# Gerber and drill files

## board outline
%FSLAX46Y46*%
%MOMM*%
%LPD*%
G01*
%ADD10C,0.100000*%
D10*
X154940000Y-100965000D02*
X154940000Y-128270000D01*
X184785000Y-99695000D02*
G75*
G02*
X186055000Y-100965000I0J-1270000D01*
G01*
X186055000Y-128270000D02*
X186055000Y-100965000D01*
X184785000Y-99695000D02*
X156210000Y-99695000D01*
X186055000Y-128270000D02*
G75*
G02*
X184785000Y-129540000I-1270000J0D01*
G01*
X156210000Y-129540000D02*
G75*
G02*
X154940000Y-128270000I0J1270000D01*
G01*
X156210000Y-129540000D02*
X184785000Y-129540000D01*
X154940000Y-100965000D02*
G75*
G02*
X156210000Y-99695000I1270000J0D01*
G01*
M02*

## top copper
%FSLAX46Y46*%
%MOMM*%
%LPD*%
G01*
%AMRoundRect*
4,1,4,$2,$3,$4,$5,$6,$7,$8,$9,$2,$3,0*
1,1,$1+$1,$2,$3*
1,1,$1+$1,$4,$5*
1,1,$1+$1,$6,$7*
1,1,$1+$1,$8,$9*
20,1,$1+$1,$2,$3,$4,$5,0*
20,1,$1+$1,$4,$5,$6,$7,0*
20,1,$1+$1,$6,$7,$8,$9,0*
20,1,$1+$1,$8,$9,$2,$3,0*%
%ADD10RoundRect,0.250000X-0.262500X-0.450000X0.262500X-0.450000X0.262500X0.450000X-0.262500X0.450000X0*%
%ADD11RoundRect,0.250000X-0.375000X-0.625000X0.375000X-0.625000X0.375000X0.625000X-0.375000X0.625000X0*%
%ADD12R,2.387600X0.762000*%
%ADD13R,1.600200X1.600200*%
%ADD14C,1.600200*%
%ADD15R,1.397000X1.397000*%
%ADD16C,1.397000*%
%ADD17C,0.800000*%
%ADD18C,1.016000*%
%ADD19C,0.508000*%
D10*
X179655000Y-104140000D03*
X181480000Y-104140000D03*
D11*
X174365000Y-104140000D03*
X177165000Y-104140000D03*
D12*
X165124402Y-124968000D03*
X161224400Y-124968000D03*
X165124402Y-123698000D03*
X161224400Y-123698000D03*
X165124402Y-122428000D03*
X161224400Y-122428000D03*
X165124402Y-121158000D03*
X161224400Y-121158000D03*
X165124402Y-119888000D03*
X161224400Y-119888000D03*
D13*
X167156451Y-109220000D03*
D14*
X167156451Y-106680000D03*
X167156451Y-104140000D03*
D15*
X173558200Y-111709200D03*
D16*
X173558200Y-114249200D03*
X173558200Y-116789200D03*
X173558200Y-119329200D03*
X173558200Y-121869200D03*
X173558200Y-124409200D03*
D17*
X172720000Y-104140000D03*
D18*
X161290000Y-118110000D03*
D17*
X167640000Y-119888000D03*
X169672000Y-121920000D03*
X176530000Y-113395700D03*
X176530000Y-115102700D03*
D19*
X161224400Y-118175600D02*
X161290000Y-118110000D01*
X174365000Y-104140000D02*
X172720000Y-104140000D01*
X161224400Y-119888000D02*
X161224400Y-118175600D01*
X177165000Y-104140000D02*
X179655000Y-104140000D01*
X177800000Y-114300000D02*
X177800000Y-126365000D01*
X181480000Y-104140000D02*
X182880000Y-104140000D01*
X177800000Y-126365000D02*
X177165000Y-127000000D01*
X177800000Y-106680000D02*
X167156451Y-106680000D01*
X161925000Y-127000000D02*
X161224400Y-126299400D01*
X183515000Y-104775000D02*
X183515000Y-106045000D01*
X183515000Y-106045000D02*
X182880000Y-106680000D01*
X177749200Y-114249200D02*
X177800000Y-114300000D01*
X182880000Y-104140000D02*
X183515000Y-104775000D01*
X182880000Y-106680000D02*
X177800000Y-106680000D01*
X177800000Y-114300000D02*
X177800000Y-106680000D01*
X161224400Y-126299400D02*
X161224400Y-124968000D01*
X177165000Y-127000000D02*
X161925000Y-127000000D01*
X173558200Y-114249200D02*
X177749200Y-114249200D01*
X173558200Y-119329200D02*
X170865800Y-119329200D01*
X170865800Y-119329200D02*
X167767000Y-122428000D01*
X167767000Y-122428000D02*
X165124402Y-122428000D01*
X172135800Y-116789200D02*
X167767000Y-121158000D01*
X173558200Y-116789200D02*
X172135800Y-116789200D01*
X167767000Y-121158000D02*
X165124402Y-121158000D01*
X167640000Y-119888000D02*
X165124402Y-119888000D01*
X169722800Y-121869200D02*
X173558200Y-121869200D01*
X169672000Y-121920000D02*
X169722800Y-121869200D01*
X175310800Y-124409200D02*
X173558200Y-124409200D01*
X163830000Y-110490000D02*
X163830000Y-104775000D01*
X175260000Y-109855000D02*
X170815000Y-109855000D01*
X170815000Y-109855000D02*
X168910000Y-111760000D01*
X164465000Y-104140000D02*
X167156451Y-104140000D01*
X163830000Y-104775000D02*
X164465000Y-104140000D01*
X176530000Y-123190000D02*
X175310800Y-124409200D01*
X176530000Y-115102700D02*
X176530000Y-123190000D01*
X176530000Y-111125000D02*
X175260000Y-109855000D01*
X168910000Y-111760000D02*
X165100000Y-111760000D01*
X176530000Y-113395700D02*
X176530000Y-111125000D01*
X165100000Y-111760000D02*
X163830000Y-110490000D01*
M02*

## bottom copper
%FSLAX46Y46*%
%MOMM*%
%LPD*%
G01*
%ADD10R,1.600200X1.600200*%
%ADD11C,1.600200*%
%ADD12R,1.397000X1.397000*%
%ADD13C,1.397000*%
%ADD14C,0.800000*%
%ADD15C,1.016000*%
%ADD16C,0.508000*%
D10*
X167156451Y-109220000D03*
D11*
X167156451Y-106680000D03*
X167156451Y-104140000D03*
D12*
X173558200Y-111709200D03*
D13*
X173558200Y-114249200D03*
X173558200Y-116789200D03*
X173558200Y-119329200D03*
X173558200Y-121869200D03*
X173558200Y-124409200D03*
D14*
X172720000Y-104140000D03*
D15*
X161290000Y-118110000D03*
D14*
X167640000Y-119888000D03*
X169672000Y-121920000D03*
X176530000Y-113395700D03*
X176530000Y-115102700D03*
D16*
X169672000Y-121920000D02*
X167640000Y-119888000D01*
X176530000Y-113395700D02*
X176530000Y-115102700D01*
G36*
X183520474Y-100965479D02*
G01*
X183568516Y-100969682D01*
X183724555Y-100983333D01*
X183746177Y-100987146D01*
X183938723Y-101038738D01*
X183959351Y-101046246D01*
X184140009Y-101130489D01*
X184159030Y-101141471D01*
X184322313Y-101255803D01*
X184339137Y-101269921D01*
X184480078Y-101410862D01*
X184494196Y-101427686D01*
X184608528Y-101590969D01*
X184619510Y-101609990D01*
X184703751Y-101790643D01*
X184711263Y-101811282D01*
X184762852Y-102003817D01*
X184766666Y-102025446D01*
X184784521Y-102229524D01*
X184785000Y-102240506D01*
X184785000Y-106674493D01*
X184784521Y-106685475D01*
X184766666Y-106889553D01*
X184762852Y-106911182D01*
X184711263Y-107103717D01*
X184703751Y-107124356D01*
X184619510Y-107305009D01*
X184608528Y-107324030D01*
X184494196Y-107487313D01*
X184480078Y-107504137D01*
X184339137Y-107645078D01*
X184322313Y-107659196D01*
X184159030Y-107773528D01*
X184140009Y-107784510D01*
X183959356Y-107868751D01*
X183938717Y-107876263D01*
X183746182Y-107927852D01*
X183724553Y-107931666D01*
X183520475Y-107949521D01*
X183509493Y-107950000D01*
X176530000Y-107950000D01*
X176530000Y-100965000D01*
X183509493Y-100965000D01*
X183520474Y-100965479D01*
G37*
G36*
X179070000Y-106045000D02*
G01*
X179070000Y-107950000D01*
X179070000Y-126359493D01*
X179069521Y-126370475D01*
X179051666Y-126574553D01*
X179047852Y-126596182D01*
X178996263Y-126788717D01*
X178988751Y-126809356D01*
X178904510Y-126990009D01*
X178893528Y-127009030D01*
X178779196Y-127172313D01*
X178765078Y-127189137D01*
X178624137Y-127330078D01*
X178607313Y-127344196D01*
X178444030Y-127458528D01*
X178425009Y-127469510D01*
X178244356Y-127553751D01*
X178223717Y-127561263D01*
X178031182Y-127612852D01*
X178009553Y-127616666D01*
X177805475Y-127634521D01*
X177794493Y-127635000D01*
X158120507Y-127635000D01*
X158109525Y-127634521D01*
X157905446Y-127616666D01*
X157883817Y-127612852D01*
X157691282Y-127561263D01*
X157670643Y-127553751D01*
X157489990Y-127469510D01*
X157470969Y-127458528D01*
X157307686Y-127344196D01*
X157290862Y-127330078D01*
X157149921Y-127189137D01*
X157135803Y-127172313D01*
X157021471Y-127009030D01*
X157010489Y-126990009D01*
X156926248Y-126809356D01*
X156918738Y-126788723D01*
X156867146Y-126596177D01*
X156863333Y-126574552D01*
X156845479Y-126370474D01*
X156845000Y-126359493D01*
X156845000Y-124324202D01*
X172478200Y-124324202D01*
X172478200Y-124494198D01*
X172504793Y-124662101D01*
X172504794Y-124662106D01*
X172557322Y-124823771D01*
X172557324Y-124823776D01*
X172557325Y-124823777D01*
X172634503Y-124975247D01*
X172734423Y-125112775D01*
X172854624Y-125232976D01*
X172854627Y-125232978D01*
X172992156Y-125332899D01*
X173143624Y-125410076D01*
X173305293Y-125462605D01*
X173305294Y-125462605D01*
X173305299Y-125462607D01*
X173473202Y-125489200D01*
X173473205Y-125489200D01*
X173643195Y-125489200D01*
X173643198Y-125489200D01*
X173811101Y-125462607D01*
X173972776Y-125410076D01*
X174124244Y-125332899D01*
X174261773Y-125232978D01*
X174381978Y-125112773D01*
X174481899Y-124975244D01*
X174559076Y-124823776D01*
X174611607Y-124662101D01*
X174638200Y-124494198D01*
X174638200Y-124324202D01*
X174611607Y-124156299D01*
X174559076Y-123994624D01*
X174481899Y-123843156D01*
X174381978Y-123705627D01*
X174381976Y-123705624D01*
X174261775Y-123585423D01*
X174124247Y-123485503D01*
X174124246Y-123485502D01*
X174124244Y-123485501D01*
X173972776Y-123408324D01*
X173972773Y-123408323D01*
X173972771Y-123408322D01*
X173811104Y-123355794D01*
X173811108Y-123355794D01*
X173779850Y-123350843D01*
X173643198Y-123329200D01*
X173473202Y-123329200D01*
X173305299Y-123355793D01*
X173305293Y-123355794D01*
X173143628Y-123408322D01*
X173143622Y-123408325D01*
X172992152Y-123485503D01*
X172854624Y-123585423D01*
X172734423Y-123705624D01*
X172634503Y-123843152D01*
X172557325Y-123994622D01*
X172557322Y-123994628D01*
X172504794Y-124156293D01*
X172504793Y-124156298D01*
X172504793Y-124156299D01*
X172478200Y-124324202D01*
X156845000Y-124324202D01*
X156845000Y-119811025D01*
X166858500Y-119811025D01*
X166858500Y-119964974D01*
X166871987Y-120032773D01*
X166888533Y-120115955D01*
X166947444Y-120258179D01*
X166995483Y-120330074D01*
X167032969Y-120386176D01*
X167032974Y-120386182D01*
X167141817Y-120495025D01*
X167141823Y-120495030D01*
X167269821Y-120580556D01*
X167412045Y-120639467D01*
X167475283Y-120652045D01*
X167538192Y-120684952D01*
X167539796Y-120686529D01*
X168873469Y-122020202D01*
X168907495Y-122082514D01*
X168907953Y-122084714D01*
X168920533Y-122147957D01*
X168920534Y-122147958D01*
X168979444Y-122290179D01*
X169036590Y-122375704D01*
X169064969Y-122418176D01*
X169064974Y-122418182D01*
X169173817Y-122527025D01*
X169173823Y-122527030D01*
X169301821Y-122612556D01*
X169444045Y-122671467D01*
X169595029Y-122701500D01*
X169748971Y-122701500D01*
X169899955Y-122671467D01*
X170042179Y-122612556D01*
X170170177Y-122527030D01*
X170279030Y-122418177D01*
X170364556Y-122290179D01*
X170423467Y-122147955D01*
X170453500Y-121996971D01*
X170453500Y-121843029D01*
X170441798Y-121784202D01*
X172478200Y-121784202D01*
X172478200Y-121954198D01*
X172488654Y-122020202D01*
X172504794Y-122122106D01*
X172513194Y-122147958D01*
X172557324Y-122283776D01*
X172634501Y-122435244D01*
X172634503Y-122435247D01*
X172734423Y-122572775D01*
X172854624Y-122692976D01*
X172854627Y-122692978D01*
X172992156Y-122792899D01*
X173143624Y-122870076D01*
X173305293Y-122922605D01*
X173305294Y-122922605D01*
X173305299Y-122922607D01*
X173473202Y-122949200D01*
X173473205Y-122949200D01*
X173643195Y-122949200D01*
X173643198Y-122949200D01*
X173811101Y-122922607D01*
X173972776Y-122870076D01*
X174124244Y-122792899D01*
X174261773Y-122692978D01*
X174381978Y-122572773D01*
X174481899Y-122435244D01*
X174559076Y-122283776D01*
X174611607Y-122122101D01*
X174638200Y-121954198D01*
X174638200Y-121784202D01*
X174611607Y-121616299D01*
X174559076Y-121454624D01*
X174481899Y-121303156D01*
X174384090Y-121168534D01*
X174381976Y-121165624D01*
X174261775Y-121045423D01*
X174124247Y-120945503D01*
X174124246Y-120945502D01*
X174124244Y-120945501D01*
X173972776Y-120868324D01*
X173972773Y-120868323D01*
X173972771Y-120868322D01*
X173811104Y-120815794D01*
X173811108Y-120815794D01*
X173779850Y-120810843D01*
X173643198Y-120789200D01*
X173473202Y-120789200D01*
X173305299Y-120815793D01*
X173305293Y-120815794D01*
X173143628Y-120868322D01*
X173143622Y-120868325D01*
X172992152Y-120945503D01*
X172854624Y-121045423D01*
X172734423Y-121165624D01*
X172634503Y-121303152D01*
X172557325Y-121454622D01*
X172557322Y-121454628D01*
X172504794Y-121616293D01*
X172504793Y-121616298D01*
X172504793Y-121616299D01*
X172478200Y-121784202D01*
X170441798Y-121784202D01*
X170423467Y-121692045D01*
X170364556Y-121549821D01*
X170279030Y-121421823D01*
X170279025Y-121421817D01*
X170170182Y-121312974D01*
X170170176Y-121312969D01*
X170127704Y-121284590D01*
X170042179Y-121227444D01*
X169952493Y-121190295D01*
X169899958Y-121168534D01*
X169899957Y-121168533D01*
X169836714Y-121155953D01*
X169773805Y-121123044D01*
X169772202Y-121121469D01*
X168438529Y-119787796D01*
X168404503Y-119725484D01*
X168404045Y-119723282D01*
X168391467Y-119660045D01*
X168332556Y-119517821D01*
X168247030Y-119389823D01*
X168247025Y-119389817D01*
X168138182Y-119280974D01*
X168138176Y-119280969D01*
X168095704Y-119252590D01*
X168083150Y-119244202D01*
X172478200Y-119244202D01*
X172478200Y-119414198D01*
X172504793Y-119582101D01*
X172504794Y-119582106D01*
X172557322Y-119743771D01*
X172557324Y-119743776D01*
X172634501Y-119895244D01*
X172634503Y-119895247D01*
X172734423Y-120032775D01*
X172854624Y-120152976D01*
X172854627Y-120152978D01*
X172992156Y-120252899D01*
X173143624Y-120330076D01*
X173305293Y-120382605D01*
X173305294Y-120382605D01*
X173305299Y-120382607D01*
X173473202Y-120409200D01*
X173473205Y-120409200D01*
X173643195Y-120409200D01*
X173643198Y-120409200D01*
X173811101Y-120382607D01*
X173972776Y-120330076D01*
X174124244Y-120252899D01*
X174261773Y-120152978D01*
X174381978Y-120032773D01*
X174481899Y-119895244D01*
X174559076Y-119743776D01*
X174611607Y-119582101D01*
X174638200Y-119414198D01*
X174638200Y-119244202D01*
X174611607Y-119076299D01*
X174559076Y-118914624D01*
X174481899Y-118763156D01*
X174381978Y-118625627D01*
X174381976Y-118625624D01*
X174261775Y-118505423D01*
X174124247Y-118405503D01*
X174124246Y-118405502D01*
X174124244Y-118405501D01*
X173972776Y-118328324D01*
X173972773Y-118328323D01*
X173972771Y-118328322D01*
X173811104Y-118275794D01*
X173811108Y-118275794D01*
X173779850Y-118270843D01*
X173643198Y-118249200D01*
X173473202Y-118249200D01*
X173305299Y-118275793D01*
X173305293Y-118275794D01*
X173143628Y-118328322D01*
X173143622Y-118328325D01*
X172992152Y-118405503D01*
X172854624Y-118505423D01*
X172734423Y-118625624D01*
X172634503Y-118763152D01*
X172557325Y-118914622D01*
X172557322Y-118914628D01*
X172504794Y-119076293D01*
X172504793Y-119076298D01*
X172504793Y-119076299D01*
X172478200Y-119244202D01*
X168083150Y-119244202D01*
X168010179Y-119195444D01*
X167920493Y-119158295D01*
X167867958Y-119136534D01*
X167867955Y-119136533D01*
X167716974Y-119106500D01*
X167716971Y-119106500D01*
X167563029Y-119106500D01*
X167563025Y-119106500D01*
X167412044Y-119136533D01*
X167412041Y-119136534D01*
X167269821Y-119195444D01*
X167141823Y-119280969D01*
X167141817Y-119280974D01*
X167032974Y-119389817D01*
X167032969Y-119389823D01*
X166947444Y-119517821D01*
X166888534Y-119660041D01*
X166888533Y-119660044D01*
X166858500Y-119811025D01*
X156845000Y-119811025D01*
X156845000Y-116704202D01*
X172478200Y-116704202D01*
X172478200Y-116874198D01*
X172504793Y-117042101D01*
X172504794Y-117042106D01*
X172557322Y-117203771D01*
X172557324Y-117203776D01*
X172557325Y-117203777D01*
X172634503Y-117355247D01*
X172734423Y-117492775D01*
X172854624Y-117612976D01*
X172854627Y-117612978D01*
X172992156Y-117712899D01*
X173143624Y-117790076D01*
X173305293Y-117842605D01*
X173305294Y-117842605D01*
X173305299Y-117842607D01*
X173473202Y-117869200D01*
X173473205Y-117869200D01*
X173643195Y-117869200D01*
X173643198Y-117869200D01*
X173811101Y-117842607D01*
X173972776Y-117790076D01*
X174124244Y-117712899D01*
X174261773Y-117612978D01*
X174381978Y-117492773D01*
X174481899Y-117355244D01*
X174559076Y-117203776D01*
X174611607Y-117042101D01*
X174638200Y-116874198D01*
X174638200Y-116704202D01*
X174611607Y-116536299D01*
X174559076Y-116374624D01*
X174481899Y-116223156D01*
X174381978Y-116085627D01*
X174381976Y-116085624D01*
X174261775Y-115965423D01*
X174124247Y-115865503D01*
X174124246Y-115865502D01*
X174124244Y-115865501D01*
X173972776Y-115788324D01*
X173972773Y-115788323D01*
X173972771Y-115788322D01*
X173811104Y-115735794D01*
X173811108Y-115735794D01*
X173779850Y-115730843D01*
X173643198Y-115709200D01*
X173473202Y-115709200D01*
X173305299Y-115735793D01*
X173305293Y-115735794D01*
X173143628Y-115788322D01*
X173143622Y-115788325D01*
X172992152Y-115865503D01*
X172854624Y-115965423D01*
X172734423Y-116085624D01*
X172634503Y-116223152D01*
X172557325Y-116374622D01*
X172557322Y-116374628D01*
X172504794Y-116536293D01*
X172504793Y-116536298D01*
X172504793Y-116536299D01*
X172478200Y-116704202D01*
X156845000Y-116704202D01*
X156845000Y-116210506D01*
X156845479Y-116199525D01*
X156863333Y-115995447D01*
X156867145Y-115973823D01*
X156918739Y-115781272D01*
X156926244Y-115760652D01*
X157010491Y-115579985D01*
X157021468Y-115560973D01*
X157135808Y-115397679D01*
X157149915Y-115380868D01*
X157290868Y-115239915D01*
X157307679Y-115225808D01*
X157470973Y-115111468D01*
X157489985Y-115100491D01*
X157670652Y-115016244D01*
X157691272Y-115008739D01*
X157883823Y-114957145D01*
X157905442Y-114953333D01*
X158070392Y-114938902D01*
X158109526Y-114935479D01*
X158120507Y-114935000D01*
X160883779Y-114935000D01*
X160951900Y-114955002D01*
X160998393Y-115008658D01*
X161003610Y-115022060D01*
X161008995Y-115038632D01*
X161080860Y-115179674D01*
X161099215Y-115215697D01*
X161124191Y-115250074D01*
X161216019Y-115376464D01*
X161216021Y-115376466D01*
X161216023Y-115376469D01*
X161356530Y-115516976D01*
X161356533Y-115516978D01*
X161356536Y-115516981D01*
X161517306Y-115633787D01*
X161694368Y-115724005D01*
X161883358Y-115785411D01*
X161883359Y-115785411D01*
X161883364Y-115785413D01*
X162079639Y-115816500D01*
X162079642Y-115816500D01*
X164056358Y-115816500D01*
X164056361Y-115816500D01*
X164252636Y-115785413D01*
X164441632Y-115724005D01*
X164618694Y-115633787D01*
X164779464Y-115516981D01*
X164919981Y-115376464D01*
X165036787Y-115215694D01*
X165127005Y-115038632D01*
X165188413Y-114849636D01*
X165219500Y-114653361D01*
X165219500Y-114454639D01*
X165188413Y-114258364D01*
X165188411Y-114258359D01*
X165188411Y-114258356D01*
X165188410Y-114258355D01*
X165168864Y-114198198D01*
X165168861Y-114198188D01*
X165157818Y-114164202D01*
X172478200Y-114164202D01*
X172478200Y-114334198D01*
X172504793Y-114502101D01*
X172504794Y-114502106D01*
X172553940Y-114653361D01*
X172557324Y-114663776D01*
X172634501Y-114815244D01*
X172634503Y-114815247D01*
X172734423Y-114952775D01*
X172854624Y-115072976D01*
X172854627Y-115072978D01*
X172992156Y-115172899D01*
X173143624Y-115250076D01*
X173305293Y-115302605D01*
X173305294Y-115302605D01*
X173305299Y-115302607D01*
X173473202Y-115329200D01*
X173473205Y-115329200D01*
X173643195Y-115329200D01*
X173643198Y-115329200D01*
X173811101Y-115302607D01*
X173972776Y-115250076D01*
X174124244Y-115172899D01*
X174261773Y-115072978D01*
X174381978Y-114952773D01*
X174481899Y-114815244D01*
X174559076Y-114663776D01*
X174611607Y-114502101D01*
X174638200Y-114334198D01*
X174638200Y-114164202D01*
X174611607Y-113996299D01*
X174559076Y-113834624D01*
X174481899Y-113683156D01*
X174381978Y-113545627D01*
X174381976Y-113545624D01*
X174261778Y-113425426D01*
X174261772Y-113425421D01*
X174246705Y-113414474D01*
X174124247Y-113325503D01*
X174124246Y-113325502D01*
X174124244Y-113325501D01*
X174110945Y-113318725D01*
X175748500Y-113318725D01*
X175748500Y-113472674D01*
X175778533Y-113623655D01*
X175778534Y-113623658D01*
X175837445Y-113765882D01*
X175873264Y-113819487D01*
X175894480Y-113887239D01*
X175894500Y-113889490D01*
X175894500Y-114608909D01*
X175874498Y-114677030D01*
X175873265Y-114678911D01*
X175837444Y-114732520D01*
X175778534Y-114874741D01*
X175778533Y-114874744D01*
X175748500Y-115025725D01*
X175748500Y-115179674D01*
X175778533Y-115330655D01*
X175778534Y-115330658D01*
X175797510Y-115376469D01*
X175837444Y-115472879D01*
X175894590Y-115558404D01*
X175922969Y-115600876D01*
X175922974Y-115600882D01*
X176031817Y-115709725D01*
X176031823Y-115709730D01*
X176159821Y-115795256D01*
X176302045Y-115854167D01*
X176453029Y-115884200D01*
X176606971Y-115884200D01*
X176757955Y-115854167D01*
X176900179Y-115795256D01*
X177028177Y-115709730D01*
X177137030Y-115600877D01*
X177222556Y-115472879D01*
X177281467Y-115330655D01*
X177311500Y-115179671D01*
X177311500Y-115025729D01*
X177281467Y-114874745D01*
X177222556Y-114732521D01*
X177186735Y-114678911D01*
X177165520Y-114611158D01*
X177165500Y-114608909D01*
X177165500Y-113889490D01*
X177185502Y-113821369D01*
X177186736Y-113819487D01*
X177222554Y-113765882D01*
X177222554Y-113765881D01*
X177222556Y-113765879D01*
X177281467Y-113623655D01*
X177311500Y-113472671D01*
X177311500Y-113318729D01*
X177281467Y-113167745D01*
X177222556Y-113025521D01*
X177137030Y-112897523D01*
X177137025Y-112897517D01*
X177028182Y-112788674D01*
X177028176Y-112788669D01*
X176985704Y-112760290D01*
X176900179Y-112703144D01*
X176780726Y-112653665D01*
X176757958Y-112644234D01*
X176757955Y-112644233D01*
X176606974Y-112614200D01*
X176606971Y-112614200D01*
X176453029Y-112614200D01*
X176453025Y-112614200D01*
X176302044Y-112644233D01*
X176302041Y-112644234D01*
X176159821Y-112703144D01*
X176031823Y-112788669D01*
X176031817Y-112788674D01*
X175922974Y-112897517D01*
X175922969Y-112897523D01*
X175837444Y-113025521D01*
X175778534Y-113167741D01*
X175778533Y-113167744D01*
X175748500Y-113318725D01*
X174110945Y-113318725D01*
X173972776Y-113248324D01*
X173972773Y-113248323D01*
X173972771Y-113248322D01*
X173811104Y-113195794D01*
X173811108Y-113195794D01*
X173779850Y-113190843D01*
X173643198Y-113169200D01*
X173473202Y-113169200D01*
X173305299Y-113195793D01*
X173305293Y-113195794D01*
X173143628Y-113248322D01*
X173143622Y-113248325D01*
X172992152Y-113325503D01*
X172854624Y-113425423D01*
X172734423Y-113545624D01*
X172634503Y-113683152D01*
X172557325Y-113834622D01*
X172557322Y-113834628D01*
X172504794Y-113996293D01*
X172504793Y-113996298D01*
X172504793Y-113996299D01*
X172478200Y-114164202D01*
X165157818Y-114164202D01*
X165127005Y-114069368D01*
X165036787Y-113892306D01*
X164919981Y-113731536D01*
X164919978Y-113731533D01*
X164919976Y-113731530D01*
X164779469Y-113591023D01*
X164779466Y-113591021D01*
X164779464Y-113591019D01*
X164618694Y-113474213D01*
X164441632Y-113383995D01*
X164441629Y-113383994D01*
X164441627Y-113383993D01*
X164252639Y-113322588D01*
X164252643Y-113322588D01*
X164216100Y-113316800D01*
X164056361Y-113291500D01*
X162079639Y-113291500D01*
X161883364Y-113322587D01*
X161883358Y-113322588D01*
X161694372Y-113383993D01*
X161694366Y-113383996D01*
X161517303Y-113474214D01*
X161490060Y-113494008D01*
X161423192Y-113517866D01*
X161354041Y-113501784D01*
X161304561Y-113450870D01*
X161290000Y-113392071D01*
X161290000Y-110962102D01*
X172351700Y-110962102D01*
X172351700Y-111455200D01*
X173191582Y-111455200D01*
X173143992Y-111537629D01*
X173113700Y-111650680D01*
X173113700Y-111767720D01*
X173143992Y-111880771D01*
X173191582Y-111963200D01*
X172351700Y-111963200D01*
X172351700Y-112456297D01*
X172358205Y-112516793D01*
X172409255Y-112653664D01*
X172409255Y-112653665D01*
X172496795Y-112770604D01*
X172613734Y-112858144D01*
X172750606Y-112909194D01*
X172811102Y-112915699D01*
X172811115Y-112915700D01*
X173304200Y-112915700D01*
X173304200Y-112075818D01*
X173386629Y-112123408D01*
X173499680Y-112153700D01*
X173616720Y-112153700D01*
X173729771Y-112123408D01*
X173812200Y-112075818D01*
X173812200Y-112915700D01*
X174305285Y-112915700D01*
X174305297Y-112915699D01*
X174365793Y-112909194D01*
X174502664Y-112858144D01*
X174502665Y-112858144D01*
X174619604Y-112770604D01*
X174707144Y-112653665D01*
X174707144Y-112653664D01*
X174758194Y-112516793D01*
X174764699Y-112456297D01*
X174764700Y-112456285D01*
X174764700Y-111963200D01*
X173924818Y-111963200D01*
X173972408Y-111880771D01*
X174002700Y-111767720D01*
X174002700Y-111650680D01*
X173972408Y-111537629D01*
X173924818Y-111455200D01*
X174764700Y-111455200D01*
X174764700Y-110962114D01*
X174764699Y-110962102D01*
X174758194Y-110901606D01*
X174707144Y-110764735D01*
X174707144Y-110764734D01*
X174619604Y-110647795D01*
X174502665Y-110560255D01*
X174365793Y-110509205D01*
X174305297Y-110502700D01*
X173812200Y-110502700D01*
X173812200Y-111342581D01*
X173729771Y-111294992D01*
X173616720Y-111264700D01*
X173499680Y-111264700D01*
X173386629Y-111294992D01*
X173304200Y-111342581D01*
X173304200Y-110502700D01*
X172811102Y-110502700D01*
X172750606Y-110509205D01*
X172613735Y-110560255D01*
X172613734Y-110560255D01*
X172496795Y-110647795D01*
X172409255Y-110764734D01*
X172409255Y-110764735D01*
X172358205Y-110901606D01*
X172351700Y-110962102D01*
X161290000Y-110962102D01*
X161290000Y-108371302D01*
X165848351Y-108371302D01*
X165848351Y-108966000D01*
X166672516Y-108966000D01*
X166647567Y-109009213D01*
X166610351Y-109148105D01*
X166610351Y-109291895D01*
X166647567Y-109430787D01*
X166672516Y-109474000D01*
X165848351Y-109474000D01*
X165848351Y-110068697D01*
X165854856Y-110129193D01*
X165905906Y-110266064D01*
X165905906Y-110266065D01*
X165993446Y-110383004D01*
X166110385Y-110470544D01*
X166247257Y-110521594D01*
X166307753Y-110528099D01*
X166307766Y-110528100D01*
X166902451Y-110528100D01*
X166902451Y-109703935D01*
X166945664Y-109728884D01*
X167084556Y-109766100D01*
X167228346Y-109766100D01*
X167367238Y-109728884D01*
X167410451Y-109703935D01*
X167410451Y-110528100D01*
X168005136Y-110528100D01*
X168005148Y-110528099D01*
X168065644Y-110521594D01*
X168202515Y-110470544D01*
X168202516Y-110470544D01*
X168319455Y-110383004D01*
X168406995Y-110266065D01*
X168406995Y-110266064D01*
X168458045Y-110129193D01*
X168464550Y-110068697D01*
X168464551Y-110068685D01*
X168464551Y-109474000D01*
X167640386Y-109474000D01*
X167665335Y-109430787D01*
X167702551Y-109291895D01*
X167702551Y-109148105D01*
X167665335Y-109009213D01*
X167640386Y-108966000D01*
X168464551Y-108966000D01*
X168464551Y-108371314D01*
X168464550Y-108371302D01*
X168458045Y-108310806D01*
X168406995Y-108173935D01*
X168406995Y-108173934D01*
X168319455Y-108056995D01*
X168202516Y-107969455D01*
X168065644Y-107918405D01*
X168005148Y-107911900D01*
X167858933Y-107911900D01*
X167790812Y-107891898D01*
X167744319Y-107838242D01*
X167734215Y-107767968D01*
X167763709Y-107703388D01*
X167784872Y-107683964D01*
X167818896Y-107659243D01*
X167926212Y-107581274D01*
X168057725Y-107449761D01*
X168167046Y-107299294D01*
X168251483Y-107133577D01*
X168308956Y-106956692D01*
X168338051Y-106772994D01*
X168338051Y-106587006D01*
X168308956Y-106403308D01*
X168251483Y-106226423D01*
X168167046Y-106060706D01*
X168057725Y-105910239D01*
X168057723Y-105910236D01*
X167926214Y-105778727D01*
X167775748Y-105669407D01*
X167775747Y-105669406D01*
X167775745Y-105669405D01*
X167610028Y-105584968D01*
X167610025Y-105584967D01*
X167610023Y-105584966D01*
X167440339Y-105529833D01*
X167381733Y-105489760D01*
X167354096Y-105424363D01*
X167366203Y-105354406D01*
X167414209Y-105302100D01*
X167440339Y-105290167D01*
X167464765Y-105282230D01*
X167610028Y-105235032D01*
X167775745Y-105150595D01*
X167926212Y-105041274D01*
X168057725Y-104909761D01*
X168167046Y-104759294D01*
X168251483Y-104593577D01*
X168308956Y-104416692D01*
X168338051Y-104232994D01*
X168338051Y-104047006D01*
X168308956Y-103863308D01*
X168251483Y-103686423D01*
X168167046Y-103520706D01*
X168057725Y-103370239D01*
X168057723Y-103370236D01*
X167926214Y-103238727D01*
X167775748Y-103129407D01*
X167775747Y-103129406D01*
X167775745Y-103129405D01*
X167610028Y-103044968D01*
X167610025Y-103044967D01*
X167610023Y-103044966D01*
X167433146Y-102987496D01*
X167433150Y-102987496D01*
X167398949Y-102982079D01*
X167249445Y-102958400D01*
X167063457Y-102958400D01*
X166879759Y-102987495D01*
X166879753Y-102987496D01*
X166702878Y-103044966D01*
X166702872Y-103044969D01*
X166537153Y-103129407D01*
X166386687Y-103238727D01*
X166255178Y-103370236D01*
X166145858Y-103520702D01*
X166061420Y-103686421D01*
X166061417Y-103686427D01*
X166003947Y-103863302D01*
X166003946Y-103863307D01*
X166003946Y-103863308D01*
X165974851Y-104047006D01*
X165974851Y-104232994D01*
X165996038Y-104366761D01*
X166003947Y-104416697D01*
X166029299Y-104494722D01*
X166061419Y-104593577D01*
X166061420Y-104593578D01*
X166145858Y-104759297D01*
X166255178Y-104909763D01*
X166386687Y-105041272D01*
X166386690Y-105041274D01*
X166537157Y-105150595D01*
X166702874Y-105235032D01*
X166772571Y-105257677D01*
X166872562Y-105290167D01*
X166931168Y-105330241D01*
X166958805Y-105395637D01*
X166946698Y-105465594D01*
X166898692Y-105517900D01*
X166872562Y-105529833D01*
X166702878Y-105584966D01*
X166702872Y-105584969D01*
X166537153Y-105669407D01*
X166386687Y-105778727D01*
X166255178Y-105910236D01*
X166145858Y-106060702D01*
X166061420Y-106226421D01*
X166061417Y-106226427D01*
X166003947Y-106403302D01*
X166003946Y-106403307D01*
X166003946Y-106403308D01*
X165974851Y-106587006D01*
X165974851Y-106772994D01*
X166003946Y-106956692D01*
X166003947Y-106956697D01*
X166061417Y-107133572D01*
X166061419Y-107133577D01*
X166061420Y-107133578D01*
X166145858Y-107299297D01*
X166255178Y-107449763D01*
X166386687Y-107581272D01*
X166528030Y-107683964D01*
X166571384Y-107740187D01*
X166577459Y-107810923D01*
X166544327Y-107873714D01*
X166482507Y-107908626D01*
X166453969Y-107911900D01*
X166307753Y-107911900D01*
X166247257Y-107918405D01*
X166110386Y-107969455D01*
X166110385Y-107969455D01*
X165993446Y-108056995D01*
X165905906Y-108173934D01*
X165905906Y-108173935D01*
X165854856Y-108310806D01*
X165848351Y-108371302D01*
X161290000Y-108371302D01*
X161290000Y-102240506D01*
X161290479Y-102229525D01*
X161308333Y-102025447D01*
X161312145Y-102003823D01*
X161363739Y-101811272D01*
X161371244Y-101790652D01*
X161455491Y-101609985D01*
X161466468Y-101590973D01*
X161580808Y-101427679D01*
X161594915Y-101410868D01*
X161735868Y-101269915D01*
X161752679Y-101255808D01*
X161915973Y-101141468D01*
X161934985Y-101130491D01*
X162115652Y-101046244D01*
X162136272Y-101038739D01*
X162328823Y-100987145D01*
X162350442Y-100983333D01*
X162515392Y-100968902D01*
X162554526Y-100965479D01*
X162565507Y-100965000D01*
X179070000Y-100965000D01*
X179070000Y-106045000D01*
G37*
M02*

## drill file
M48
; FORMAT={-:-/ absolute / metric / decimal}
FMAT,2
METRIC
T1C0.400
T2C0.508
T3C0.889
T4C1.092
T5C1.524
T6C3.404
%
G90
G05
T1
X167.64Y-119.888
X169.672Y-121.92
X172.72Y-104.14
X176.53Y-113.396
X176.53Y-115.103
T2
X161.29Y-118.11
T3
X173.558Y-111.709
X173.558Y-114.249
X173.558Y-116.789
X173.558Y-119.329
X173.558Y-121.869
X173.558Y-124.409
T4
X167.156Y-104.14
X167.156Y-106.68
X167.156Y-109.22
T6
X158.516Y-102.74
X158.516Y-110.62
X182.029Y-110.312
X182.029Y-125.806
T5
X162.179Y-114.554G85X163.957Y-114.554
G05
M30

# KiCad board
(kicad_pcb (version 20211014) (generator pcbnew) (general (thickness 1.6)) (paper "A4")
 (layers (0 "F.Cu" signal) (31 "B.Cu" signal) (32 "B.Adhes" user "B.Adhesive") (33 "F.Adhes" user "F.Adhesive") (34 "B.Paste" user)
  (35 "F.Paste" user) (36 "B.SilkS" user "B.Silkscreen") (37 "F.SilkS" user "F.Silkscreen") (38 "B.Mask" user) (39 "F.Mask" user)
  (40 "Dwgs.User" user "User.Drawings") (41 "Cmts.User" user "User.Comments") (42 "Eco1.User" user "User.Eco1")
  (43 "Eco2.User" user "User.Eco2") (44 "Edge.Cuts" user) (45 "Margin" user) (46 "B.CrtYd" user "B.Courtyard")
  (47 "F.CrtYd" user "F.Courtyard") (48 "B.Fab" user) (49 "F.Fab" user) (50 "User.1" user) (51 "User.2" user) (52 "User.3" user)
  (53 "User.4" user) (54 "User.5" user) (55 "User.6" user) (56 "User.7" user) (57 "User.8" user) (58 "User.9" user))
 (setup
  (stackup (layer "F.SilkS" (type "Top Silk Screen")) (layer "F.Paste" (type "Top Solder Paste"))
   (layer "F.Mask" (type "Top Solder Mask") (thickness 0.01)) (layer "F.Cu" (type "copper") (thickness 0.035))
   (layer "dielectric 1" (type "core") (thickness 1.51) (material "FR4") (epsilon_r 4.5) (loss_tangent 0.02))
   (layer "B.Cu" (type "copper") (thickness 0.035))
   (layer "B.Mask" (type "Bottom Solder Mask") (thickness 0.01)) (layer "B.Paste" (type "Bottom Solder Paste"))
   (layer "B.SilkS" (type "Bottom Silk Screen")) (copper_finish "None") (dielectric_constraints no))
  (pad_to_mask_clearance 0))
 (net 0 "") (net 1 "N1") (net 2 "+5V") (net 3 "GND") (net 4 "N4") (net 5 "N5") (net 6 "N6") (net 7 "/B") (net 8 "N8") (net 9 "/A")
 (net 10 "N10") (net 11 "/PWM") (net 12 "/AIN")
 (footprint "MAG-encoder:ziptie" (layer "F.Cu") (at 163.068 114.554)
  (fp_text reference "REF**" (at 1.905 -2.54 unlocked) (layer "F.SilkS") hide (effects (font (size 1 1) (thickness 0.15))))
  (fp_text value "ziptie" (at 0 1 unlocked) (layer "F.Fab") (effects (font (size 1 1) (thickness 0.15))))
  (pad "" np_thru_hole oval (at 0 0) (size 3.302 1.524) (drill oval 3.302 1.524) (layers F&B.Cu *.Mask)))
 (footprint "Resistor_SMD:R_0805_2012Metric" (layer "F.Cu") (at 180.5675 104.14)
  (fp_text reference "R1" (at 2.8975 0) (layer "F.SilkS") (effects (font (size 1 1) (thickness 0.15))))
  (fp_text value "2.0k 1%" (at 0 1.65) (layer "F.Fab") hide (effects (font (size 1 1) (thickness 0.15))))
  (pad "1" smd roundrect (at -0.9125 0) (size 1.025 1.4) (layers "F.Cu" "F.Paste" "F.Mask") (roundrect_rratio 0.243902) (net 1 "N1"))
  (pad "2" smd roundrect (at 0.9125 0) (size 1.025 1.4) (layers "F.Cu" "F.Paste" "F.Mask") (roundrect_rratio 0.243902) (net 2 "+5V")))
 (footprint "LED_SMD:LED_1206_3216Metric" (layer "F.Cu") (at 175.765 104.14)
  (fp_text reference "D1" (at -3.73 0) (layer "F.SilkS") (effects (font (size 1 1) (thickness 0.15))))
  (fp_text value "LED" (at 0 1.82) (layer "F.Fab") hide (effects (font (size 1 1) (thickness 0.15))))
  (pad "1" smd roundrect (at -1.4 0) (size 1.25 1.75) (layers "F.Cu" "F.Paste" "F.Mask") (roundrect_rratio 0.2) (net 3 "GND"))
  (pad "2" smd roundrect (at 1.4 0) (size 1.25 1.75) (layers "F.Cu" "F.Paste" "F.Mask") (roundrect_rratio 0.2) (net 1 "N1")))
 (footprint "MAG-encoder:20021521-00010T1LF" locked (layer "F.Cu") (at 163.174401 122.428 90)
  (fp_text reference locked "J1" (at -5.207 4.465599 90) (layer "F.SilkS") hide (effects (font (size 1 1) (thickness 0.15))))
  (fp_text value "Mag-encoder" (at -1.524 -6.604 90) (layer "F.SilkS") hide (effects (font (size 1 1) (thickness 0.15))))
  (pad "1" smd rect locked (at -2.54 1.950001 90) (size 0.762 2.3876) (layers "F.Cu" "F.Paste" "F.Mask") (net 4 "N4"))
  (pad "2" smd rect locked (at -2.54 -1.950001 90) (size 0.762 2.3876) (layers "F.Cu" "F.Paste" "F.Mask") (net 2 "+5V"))
  (pad "3" smd rect locked (at -1.27 1.950001 90) (size 0.762 2.3876) (layers "F.Cu" "F.Paste" "F.Mask") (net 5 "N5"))
  (pad "4" smd rect locked (at -1.27 -1.950001 90) (size 0.762 2.3876) (layers "F.Cu" "F.Paste" "F.Mask") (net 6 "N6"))
  (pad "5" smd rect locked (at 0 1.950001 90) (size 0.762 2.3876) (layers "F.Cu" "F.Paste" "F.Mask") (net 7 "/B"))
  (pad "6" smd rect locked (at 0 -1.950001 90) (size 0.762 2.3876) (layers "F.Cu" "F.Paste" "F.Mask") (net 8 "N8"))
  (pad "7" smd rect locked (at 1.27 1.950001 90) (size 0.762 2.3876) (layers "F.Cu" "F.Paste" "F.Mask") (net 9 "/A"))
  (pad "8" smd rect locked (at 1.27 -1.950001 90) (size 0.762 2.3876) (layers "F.Cu" "F.Paste" "F.Mask") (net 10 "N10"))
  (pad "9" smd rect locked (at 2.54 1.950001 90) (size 0.762 2.3876) (layers "F.Cu" "F.Paste" "F.Mask") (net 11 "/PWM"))
  (pad "10" smd rect locked (at 2.54 -1.950001 90) (size 0.762 2.3876) (layers "F.Cu" "F.Paste" "F.Mask") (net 3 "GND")))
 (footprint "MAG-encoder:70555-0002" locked (layer "B.Cu") (at 167.156451 109.22 90)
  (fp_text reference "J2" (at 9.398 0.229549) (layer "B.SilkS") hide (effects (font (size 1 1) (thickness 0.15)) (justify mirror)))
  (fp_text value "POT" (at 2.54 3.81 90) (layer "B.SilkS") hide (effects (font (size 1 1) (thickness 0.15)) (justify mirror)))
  (pad "" np_thru_hole circle locked (at 6.48 -8.640001 90) (size 3.4036 3.4036) (drill 3.4036) (layers *.Cu *.Mask))
  (pad "" np_thru_hole circle locked (at -1.4 -8.640001 90) (size 3.4036 3.4036) (drill 3.4036) (layers *.Cu *.Mask))
  (pad "1" thru_hole rect locked (at 0 0 90) (size 1.6002 1.6002) (drill 1.0922) (layers *.Cu *.Mask) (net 3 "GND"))
  (pad "2" thru_hole circle locked (at 2.54 0 90) (size 1.6002 1.6002) (drill 1.0922) (layers *.Cu *.Mask) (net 2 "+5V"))
  (pad "3" thru_hole circle locked (at 5.08 0 90) (size 1.6002 1.6002) (drill 1.0922) (layers *.Cu *.Mask) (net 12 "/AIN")))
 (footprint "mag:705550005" (layer "B.Cu") (at 173.5582 111.7092 -90)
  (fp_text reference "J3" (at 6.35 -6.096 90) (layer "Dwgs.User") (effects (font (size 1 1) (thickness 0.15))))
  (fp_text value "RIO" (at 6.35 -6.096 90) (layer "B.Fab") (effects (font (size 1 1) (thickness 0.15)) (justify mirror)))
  (pad "" np_thru_hole circle (at -1.397 -8.4709 180) (size 3.4036 3.4036) (drill 3.4036) (layers F&B.Cu *.Mask))
  (pad "" np_thru_hole circle (at 14.097 -8.4709 180) (size 3.4036 3.4036) (drill 3.4036) (layers F&B.Cu *.Mask))
  (pad "1" thru_hole rect (at 0 0 270) (size 1.397 1.397) (drill 0.889) (layers *.Cu *.Mask) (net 3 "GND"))
  (pad "2" thru_hole circle (at 2.54 0 270) (size 1.397 1.397) (drill 0.889) (layers *.Cu *.Mask) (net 2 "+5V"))
  (pad "3" thru_hole circle (at 5.08 0 270) (size 1.397 1.397) (drill 0.889) (layers *.Cu *.Mask) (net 9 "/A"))
  (pad "4" thru_hole circle (at 7.62 0 270) (size 1.397 1.397) (drill 0.889) (layers *.Cu *.Mask) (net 7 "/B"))
  (pad "5" thru_hole circle (at 10.16 0 270) (size 1.397 1.397) (drill 0.889) (layers *.Cu *.Mask) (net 11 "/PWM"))
  (pad "6" thru_hole circle (at 12.7 0 270) (size 1.397 1.397) (drill 0.889) (layers *.Cu *.Mask) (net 12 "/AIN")))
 (gr_line (start 154.94 100.965) (end 154.94 128.27) (layer "Edge.Cuts") (width 0.1))
 (gr_arc (start 184.785 99.695) (mid 185.683026 100.066974) (end 186.055 100.965) (layer "Edge.Cuts") (width 0.1))
 (gr_line (start 186.055 128.27) (end 186.055 100.965) (layer "Edge.Cuts") (width 0.1))
 (gr_line (start 184.785 99.695) (end 156.21 99.695) (layer "Edge.Cuts") (width 0.1))
 (gr_arc (start 186.055 128.27) (mid 185.683026 129.168026) (end 184.785 129.54) (layer "Edge.Cuts") (width 0.1))
 (gr_arc (start 156.21 129.54) (mid 155.311974 129.168026) (end 154.94 128.27) (layer "Edge.Cuts") (width 0.1))
 (gr_line (start 156.21 129.54) (end 184.785 129.54) (layer "Edge.Cuts") (width 0.1))
 (gr_arc (start 154.94 100.965) (mid 155.311974 100.066974) (end 156.21 99.695) (layer "Edge.Cuts") (width 0.1))
 (segment (start 161.2244 118.1756) (end 161.29 118.11) (width 0.508) (layer "F.Cu") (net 3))
 (segment (start 174.365 104.14) (end 172.72 104.14) (width 0.508) (layer "F.Cu") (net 3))
 (segment (start 161.2244 119.888) (end 161.2244 118.1756) (width 0.508) (layer "F.Cu") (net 3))
 (via (at 172.72 104.14) (size 0.8) (drill 0.4) (layers "F.Cu" "B.Cu") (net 3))
 (via (at 161.29 118.11) (size 1.016) (drill 0.508) (layers "F.Cu" "B.Cu") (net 3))
 (segment (start 177.165 104.14) (end 179.655 104.14) (width 0.508) (layer "F.Cu") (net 1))
 (segment (start 177.8 114.3) (end 177.8 126.365) (width 0.508) (layer "F.Cu") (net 2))
 (segment (start 181.48 104.14) (end 182.88 104.14) (width 0.508) (layer "F.Cu") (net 2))
 (segment (start 177.8 126.365) (end 177.165 127) (width 0.508) (layer "F.Cu") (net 2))
 (segment (start 177.8 106.68) (end 167.156451 106.68) (width 0.508) (layer "F.Cu") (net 2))
 (segment (start 161.925 127) (end 161.2244 126.2994) (width 0.508) (layer "F.Cu") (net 2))
 (segment (start 183.515 104.775) (end 183.515 106.045) (width 0.508) (layer "F.Cu") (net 2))
 (segment (start 183.515 106.045) (end 182.88 106.68) (width 0.508) (layer "F.Cu") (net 2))
 (segment (start 177.7492 114.2492) (end 177.8 114.3) (width 0.508) (layer "F.Cu") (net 2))
 (segment (start 182.88 104.14) (end 183.515 104.775) (width 0.508) (layer "F.Cu") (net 2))
 (segment (start 182.88 106.68) (end 177.8 106.68) (width 0.508) (layer "F.Cu") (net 2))
 (segment (start 177.8 114.3) (end 177.8 106.68) (width 0.508) (layer "F.Cu") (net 2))
 (segment (start 161.2244 126.2994) (end 161.2244 124.968) (width 0.508) (layer "F.Cu") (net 2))
 (segment (start 177.165 127) (end 161.925 127) (width 0.508) (layer "F.Cu") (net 2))
 (segment (start 173.5582 114.2492) (end 177.7492 114.2492) (width 0.508) (layer "F.Cu") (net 2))
 (segment (start 173.5582 119.3292) (end 170.8658 119.3292) (width 0.508) (layer "F.Cu") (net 7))
 (segment (start 170.8658 119.3292) (end 167.767 122.428) (width 0.508) (layer "F.Cu") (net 7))
 (segment (start 167.767 122.428) (end 165.124402 122.428) (width 0.508) (layer "F.Cu") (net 7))
 (segment (start 172.1358 116.7892) (end 167.767 121.158) (width 0.508) (layer "F.Cu") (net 9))
 (segment (start 173.5582 116.7892) (end 172.1358 116.7892) (width 0.508) (layer "F.Cu") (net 9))
 (segment (start 167.767 121.158) (end 165.124402 121.158) (width 0.508) (layer "F.Cu") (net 9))
 (segment (start 167.64 119.888) (end 165.124402 119.888) (width 0.508) (layer "F.Cu") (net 11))
 (segment (start 169.7228 121.8692) (end 173.5582 121.8692) (width 0.508) (layer "F.Cu") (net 11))
 (segment (start 169.672 121.92) (end 169.7228 121.8692) (width 0.508) (layer "F.Cu") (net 11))
 (via (at 167.64 119.888) (size 0.8) (drill 0.4) (layers "F.Cu" "B.Cu") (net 11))
 (via (at 169.672 121.92) (size 0.8) (drill 0.4) (layers "F.Cu" "B.Cu") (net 11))
 (segment (start 169.672 121.92) (end 167.64 119.888) (width 0.508) (layer "B.Cu") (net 11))
 (segment (start 175.3108 124.4092) (end 173.5582 124.4092) (width 0.508) (layer "F.Cu") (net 12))
 (segment (start 163.83 110.49) (end 163.83 104.775) (width 0.508) (layer "F.Cu") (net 12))
 (segment (start 175.26 109.855) (end 170.815 109.855) (width 0.508) (layer "F.Cu") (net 12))
 (segment (start 170.815 109.855) (end 168.91 111.76) (width 0.508) (layer "F.Cu") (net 12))
 (segment (start 164.465 104.14) (end 167.156451 104.14) (width 0.508) (layer "F.Cu") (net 12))
 (segment (start 163.83 104.775) (end 164.465 104.14) (width 0.508) (layer "F.Cu") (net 12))
 (segment (start 176.53 123.19) (end 175.3108 124.4092) (width 0.508) (layer "F.Cu") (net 12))
 (segment (start 176.53 115.1027) (end 176.53 123.19) (width 0.508) (layer "F.Cu") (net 12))
 (segment (start 176.53 111.125) (end 175.26 109.855) (width 0.508) (layer "F.Cu") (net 12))
 (segment (start 168.91 111.76) (end 165.1 111.76) (width 0.508) (layer "F.Cu") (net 12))
 (segment (start 176.53 113.3957) (end 176.53 111.125) (width 0.508) (layer "F.Cu") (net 12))
 (segment (start 165.1 111.76) (end 163.83 110.49) (width 0.508) (layer "F.Cu") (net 12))
 (via (at 176.53 113.3957) (size 0.8) (drill 0.4) (layers "F.Cu" "B.Cu") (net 12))
 (via (at 176.53 115.1027) (size 0.8) (drill 0.4) (layers "F.Cu" "B.Cu") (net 12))
 (segment (start 176.53 113.3957) (end 176.53 115.1027) (width 0.508) (layer "B.Cu") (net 12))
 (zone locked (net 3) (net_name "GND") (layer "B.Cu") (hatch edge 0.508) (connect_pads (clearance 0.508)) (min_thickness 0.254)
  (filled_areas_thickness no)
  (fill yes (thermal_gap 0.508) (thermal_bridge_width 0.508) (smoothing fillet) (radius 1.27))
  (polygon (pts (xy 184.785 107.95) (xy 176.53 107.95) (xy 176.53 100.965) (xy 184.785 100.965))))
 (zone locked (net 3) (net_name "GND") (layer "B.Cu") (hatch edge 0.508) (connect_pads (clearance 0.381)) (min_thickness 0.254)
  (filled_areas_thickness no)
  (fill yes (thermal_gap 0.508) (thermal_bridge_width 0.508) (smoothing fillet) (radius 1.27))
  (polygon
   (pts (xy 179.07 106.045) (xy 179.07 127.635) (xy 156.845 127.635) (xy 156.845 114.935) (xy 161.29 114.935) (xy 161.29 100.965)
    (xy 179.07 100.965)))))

